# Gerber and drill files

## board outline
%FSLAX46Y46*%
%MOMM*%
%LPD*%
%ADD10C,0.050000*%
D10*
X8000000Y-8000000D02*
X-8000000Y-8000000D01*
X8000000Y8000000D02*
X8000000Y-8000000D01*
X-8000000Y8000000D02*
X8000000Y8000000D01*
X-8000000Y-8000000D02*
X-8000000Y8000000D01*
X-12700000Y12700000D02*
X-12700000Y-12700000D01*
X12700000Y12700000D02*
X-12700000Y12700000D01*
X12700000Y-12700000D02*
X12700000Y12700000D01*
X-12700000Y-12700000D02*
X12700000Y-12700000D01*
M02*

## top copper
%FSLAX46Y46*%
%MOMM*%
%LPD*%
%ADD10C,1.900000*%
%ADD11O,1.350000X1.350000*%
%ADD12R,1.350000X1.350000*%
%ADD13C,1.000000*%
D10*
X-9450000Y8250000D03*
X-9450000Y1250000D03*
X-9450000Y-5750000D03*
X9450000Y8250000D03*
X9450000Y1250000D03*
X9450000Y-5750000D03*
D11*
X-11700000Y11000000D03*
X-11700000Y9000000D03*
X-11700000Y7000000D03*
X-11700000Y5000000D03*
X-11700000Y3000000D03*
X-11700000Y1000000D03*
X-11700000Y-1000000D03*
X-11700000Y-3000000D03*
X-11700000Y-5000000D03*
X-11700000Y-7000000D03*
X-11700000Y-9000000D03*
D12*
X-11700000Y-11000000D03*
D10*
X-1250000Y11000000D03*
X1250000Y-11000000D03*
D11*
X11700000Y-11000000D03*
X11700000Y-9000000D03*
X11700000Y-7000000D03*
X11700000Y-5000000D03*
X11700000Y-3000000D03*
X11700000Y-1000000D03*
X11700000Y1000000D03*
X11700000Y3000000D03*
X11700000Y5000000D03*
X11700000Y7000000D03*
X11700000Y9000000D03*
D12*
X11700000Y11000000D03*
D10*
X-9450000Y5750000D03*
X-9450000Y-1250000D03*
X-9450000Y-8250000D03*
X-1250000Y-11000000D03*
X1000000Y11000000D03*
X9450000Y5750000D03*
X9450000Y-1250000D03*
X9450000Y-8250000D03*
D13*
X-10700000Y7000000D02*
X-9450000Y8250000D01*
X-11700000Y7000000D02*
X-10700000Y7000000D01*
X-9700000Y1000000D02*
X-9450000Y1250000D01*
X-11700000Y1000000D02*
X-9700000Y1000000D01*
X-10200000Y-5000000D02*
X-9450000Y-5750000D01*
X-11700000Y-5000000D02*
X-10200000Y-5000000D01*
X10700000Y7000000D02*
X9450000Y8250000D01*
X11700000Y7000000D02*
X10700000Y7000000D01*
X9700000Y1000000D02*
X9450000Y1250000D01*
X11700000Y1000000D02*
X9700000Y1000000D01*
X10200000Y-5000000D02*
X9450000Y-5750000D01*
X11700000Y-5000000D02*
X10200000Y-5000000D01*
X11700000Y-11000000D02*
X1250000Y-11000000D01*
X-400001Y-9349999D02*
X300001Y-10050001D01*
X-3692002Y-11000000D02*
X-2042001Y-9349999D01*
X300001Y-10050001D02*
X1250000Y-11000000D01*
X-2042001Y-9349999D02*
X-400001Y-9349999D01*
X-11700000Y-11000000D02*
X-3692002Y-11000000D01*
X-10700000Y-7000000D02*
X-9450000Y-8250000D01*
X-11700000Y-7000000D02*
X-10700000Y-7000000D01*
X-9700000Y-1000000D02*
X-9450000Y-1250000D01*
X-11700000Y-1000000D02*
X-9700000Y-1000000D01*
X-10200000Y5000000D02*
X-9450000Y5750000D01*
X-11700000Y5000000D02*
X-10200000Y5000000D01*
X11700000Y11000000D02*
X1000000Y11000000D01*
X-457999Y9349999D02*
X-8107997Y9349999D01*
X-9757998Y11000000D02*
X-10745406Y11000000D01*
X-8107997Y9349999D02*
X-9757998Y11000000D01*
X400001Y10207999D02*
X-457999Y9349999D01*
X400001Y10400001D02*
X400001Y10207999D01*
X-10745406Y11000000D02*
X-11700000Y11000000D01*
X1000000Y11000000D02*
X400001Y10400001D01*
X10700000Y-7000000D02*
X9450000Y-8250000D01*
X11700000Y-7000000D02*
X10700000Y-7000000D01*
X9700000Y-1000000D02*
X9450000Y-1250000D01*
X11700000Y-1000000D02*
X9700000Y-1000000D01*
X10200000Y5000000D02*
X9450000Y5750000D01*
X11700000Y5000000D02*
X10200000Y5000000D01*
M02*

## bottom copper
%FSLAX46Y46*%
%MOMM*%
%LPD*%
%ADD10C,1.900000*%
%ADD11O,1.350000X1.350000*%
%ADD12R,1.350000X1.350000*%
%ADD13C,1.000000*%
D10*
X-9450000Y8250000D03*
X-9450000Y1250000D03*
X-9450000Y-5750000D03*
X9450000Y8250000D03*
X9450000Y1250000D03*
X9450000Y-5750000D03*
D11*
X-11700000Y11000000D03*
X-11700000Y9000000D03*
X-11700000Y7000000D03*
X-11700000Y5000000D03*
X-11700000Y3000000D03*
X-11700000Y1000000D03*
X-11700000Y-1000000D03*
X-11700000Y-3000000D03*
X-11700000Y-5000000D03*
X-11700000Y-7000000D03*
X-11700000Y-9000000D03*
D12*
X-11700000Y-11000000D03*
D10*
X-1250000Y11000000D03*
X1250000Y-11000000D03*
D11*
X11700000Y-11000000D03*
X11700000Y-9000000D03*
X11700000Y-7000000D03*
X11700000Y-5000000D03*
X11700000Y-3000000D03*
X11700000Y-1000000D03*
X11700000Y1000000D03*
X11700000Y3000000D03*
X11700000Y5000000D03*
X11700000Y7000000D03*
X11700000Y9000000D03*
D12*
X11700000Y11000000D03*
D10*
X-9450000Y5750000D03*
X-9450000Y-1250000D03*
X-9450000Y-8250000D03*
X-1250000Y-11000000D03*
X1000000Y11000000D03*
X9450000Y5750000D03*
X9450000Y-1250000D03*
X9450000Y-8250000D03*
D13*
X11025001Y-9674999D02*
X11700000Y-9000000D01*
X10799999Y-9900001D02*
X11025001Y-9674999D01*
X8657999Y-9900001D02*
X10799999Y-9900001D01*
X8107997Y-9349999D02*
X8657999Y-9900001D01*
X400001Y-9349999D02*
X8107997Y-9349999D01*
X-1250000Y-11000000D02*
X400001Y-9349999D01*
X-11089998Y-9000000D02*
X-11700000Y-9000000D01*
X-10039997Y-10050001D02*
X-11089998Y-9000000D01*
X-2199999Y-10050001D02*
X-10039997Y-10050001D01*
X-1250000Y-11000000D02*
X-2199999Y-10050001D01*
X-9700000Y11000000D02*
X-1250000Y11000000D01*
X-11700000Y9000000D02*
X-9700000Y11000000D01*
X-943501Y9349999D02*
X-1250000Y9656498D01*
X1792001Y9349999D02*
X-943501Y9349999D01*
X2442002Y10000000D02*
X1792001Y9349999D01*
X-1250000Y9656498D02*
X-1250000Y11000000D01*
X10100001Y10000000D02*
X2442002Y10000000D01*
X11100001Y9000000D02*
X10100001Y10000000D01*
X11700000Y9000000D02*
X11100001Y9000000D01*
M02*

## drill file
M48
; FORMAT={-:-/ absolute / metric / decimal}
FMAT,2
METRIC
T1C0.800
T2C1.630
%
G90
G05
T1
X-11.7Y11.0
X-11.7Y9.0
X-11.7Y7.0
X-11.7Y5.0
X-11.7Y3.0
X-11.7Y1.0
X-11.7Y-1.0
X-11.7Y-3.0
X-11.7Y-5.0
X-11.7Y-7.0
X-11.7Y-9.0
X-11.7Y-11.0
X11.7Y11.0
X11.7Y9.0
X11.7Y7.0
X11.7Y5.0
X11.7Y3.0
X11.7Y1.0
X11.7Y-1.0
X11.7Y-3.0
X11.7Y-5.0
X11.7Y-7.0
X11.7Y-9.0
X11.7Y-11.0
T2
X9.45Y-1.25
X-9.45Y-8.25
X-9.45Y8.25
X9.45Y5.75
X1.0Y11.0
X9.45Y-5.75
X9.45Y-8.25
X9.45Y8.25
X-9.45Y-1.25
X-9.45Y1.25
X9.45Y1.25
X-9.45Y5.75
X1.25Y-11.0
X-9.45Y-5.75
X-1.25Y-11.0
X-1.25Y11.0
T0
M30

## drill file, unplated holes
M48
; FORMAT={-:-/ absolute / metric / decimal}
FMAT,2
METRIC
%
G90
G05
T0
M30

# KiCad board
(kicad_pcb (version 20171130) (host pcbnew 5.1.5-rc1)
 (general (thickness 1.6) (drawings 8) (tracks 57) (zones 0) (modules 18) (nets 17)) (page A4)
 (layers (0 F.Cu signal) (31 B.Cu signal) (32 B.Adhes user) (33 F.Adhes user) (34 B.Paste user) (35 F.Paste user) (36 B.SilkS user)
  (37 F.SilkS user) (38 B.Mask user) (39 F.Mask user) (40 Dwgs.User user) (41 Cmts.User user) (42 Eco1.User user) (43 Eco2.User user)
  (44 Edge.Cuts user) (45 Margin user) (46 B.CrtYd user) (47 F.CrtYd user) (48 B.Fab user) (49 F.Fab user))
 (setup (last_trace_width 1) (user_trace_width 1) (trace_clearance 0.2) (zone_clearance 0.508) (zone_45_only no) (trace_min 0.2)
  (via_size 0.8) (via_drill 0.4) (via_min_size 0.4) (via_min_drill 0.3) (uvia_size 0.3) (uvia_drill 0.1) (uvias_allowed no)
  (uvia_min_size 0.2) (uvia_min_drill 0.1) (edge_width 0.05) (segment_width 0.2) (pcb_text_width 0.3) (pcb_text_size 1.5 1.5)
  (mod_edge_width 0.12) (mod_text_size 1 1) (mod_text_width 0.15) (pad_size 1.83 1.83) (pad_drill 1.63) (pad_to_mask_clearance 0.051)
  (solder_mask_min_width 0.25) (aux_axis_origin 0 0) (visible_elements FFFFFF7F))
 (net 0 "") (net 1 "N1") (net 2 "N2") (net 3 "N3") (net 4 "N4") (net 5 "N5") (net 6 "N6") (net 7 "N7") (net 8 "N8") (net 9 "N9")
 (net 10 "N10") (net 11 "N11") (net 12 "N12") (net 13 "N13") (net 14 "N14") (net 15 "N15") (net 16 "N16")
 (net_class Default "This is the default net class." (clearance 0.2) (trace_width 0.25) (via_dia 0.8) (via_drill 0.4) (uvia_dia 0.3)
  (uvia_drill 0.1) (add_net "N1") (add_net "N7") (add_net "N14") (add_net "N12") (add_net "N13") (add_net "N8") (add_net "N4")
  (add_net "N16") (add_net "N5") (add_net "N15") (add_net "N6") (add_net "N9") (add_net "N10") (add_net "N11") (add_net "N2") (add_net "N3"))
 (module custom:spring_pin (layer F.Cu) (at -9.45 -8.25 90)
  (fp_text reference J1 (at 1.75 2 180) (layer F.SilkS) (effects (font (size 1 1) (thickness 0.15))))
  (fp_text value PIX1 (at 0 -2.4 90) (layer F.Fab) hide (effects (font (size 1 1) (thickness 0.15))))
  (pad 1 thru_hole circle (at 0 0 90) (size 1.9 1.9) (drill 1.63) (layers *.Cu *.Mask) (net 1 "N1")))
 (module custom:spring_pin (layer F.Cu) (at -9.45 -1.25 90)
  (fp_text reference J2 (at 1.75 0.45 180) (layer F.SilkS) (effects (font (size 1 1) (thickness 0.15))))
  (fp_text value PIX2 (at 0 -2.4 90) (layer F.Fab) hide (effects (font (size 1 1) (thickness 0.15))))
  (pad 1 thru_hole circle (at 0 0 90) (size 1.9 1.9) (drill 1.63) (layers *.Cu *.Mask) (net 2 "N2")))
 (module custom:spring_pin (layer F.Cu) (at -9.45 5.75 90)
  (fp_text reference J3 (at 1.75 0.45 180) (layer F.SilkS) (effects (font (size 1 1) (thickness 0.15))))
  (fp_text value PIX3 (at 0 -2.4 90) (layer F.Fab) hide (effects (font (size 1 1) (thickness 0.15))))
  (pad 1 thru_hole circle (at 0 0 90) (size 1.9 1.9) (drill 1.63) (layers *.Cu *.Mask) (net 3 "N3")))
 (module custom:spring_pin (layer F.Cu) (at 9.45 -8.25 90)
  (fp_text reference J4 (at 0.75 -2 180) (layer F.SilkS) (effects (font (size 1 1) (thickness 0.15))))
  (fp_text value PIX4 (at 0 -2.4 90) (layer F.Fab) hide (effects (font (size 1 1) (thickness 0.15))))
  (pad 1 thru_hole circle (at 0 0 90) (size 1.9 1.9) (drill 1.63) (layers *.Cu *.Mask) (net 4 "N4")))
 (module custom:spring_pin (layer F.Cu) (at 9.45 -1.25 90)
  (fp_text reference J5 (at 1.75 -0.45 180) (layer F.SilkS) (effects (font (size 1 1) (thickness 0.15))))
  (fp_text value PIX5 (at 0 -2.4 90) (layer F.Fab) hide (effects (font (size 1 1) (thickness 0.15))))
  (pad 1 thru_hole circle (at 0 0 90) (size 1.9 1.9) (drill 1.63) (layers *.Cu *.Mask) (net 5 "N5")))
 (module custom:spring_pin (layer F.Cu) (at 9.45 5.75 90)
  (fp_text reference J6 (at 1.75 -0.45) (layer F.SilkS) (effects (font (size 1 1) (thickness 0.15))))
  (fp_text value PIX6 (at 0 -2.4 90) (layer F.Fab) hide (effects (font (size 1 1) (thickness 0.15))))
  (pad 1 thru_hole circle (at 0 0 90) (size 1.9 1.9) (drill 1.63) (layers *.Cu *.Mask) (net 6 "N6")))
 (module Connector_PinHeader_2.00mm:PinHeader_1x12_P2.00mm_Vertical (layer B.Cu) (at -11.7 11)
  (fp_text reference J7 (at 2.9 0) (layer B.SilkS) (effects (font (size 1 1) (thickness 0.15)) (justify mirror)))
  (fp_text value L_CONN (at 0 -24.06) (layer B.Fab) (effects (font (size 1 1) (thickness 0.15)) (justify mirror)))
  (pad 12 thru_hole oval (at 0 -22) (size 1.35 1.35) (drill 0.8) (layers *.Cu *.Mask) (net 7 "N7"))
  (pad 11 thru_hole oval (at 0 -20) (size 1.35 1.35) (drill 0.8) (layers *.Cu *.Mask) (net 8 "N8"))
  (pad 10 thru_hole oval (at 0 -18) (size 1.35 1.35) (drill 0.8) (layers *.Cu *.Mask) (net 1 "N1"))
  (pad 9 thru_hole oval (at 0 -16) (size 1.35 1.35) (drill 0.8) (layers *.Cu *.Mask) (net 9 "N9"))
  (pad 8 thru_hole oval (at 0 -14) (size 1.35 1.35) (drill 0.8) (layers *.Cu *.Mask))
  (pad 7 thru_hole oval (at 0 -12) (size 1.35 1.35) (drill 0.8) (layers *.Cu *.Mask) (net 2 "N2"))
  (pad 6 thru_hole oval (at 0 -10) (size 1.35 1.35) (drill 0.8) (layers *.Cu *.Mask) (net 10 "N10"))
  (pad 5 thru_hole oval (at 0 -8) (size 1.35 1.35) (drill 0.8) (layers *.Cu *.Mask))
  (pad 4 thru_hole oval (at 0 -6) (size 1.35 1.35) (drill 0.8) (layers *.Cu *.Mask) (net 3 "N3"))
  (pad 3 thru_hole oval (at 0 -4) (size 1.35 1.35) (drill 0.8) (layers *.Cu *.Mask) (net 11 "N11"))
  (pad 2 thru_hole oval (at 0 -2) (size 1.35 1.35) (drill 0.8) (layers *.Cu *.Mask) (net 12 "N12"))
  (pad 1 thru_hole rect (at 0 0) (size 1.35 1.35) (drill 0.8) (layers *.Cu *.Mask) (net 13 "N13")))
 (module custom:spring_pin (layer F.Cu) (at -1.25 -11 90)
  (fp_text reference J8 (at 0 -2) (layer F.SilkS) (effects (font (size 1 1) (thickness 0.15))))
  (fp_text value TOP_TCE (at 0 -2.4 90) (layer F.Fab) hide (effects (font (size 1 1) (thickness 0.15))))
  (pad 1 thru_hole circle (at 0 0 90) (size 1.9 1.9) (drill 1.63) (layers *.Cu *.Mask) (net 8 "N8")))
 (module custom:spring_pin (layer F.Cu) (at 1.25 11 90)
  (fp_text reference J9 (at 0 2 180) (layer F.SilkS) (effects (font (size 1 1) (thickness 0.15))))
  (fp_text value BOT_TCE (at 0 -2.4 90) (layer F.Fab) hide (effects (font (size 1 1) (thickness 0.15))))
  (pad 1 thru_hole circle (at 0 0 90) (size 1.9 1.9) (drill 1.63) (layers *.Cu *.Mask) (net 13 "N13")))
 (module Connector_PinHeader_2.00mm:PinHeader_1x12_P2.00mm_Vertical (layer B.Cu) (at 11.7 -11 180)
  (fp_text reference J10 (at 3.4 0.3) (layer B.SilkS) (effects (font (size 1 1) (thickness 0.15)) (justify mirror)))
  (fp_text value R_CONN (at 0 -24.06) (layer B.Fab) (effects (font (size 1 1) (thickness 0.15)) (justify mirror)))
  (pad 12 thru_hole oval (at 0 -22 180) (size 1.35 1.35) (drill 0.8) (layers *.Cu *.Mask) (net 13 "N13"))
  (pad 11 thru_hole oval (at 0 -20 180) (size 1.35 1.35) (drill 0.8) (layers *.Cu *.Mask) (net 12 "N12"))
  (pad 10 thru_hole oval (at 0 -18 180) (size 1.35 1.35) (drill 0.8) (layers *.Cu *.Mask) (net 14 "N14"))
  (pad 9 thru_hole oval (at 0 -16 180) (size 1.35 1.35) (drill 0.8) (layers *.Cu *.Mask) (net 6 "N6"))
  (pad 8 thru_hole oval (at 0 -14 180) (size 1.35 1.35) (drill 0.8) (layers *.Cu *.Mask))
  (pad 7 thru_hole oval (at 0 -12 180) (size 1.35 1.35) (drill 0.8) (layers *.Cu *.Mask) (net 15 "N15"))
  (pad 6 thru_hole oval (at 0 -10 180) (size 1.35 1.35) (drill 0.8) (layers *.Cu *.Mask) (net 5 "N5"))
  (pad 5 thru_hole oval (at 0 -8 180) (size 1.35 1.35) (drill 0.8) (layers *.Cu *.Mask))
  (pad 4 thru_hole oval (at 0 -6 180) (size 1.35 1.35) (drill 0.8) (layers *.Cu *.Mask) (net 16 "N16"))
  (pad 3 thru_hole oval (at 0 -4 180) (size 1.35 1.35) (drill 0.8) (layers *.Cu *.Mask) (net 4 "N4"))
  (pad 2 thru_hole oval (at 0 -2 180) (size 1.35 1.35) (drill 0.8) (layers *.Cu *.Mask) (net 8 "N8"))
  (pad 1 thru_hole rect (at 0 0 180) (size 1.35 1.35) (drill 0.8) (layers *.Cu *.Mask) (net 7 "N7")))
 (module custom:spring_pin (layer F.Cu) (at -9.45 -5.75 90)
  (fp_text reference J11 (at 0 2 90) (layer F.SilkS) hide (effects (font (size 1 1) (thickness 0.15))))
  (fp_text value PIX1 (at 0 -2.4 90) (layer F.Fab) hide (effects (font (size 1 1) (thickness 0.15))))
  (pad 1 thru_hole circle (at 0 0 90) (size 1.9 1.9) (drill 1.63) (layers *.Cu *.Mask) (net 9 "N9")))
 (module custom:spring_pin (layer F.Cu) (at -9.45 1.25 90)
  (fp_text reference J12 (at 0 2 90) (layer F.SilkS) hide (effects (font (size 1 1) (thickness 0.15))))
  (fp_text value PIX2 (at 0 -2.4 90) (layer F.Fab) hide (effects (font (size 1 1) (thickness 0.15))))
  (pad 1 thru_hole circle (at 0 0 90) (size 1.9 1.9) (drill 1.63) (layers *.Cu *.Mask) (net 10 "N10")))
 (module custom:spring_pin (layer F.Cu) (at -9.45 8.25 90)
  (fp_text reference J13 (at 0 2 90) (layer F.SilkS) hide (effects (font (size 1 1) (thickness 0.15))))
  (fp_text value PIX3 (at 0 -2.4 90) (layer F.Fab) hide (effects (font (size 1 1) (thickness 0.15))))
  (pad 1 thru_hole circle (at 0 0 90) (size 1.9 1.9) (drill 1.63) (layers *.Cu *.Mask) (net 11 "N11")))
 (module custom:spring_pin (layer F.Cu) (at -1.25 11 90)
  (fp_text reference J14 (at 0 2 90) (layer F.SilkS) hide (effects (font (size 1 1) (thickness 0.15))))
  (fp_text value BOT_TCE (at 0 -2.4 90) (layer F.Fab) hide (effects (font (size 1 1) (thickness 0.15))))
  (pad 1 thru_hole circle (at 0 0 90) (size 1.9 1.9) (drill 1.63) (layers *.Cu *.Mask) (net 12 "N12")))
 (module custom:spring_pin (layer F.Cu) (at 1 -11 90)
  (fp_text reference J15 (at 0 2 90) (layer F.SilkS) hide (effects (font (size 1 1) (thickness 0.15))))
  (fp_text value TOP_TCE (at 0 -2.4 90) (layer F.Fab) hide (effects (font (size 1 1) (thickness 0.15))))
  (pad 1 thru_hole circle (at 0 0 90) (size 1.9 1.9) (drill 1.63) (layers *.Cu *.Mask) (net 7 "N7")))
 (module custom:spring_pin (layer F.Cu) (at 9.45 -5.75 90)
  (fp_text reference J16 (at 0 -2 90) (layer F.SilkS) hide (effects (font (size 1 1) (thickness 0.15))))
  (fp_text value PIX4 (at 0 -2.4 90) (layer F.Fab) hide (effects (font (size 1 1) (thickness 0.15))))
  (pad 1 thru_hole circle (at 0 0 90) (size 1.9 1.9) (drill 1.63) (layers *.Cu *.Mask) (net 16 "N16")))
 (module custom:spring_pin (layer F.Cu) (at 9.45 1.25 90)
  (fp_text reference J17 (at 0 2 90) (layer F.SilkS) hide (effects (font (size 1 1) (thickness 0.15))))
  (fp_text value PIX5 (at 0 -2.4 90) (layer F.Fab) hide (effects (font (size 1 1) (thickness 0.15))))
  (pad 1 thru_hole circle (at 0 0 90) (size 1.9 1.9) (drill 1.63) (layers *.Cu *.Mask) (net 15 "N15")))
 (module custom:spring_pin (layer F.Cu) (at 9.45 8.25 90)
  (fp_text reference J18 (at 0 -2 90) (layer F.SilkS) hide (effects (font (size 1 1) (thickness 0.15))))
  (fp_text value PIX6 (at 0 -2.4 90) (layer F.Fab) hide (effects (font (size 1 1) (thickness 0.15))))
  (pad 1 thru_hole circle (at 0 0 90) (size 1.9 1.9) (drill 1.63) (layers *.Cu *.Mask) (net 14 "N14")))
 (gr_line (start 8 8) (end -8 8) (layer Edge.Cuts) (width 0.05))
 (gr_line (start 8 -8) (end 8 8) (layer Edge.Cuts) (width 0.05))
 (gr_line (start -8 -8) (end 8 -8) (layer Edge.Cuts) (width 0.05))
 (gr_line (start -8 8) (end -8 -8) (layer Edge.Cuts) (width 0.05))
 (gr_line (start -12.7 -12.7) (end -12.7 12.7) (layer Edge.Cuts) (width 0.05))
 (gr_line (start 12.7 -12.7) (end -12.7 -12.7) (layer Edge.Cuts) (width 0.05))
 (gr_line (start 12.7 12.7) (end 12.7 -12.7) (layer Edge.Cuts) (width 0.05))
 (gr_line (start -12.7 12.7) (end 12.7 12.7) (layer Edge.Cuts) (width 0.05))
 (segment (start -10.7 -7) (end -9.45 -8.25) (width 1) (layer F.Cu) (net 1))
 (segment (start -11.7 -7) (end -10.7 -7) (width 1) (layer F.Cu) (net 1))
 (segment (start -9.7 -1) (end -9.45 -1.25) (width 1) (layer F.Cu) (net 2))
 (segment (start -11.7 -1) (end -9.7 -1) (width 1) (layer F.Cu) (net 2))
 (segment (start -10.2 5) (end -9.45 5.75) (width 1) (layer F.Cu) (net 3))
 (segment (start -11.7 5) (end -10.2 5) (width 1) (layer F.Cu) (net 3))
 (segment (start 10.7 -7) (end 9.45 -8.25) (width 1) (layer F.Cu) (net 4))
 (segment (start 11.7 -7) (end 10.7 -7) (width 1) (layer F.Cu) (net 4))
 (segment (start 9.7 -1) (end 9.45 -1.25) (width 1) (layer F.Cu) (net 5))
 (segment (start 11.7 -1) (end 9.7 -1) (width 1) (layer F.Cu) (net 5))
 (segment (start 10.2 5) (end 9.45 5.75) (width 1) (layer F.Cu) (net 6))
 (segment (start 11.7 5) (end 10.2 5) (width 1) (layer F.Cu) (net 6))
 (segment (start 11.7 11) (end 1.25 11) (width 1) (layer F.Cu) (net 13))
 (segment (start -0.400001 9.349999) (end 0.300001 10.050001) (width 1) (layer F.Cu) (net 13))
 (segment (start -3.692002 11) (end -2.042001 9.349999) (width 1) (layer F.Cu) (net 13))
 (segment (start 0.300001 10.050001) (end 1.25 11) (width 1) (layer F.Cu) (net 13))
 (segment (start -2.042001 9.349999) (end -0.400001 9.349999) (width 1) (layer F.Cu) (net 13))
 (segment (start -11.7 11) (end -3.692002 11) (width 1) (layer F.Cu) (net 13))
 (segment (start 11.025001 9.674999) (end 11.7 9) (width 1) (layer B.Cu) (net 12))
 (segment (start 10.799999 9.900001) (end 11.025001 9.674999) (width 1) (layer B.Cu) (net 12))
 (segment (start 8.657999 9.900001) (end 10.799999 9.900001) (width 1) (layer B.Cu) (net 12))
 (segment (start 8.107997 9.349999) (end 8.657999 9.900001) (width 1) (layer B.Cu) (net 12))
 (segment (start 0.400001 9.349999) (end 8.107997 9.349999) (width 1) (layer B.Cu) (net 12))
 (segment (start -1.25 11) (end 0.400001 9.349999) (width 1) (layer B.Cu) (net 12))
 (segment (start -11.089998 9) (end -11.7 9) (width 1) (layer B.Cu) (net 12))
 (segment (start -10.039997 10.050001) (end -11.089998 9) (width 1) (layer B.Cu) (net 12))
 (segment (start -2.199999 10.050001) (end -10.039997 10.050001) (width 1) (layer B.Cu) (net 12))
 (segment (start -1.25 11) (end -2.199999 10.050001) (width 1) (layer B.Cu) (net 12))
 (segment (start -10.7 7) (end -9.45 8.25) (width 1) (layer F.Cu) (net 11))
 (segment (start -11.7 7) (end -10.7 7) (width 1) (layer F.Cu) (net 11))
 (segment (start -9.7 1) (end -9.45 1.25) (width 1) (layer F.Cu) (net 10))
 (segment (start -11.7 1) (end -9.7 1) (width 1) (layer F.Cu) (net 10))
 (segment (start -10.2 -5) (end -9.45 -5.75) (width 1) (layer F.Cu) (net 9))
 (segment (start -11.7 -5) (end -10.2 -5) (width 1) (layer F.Cu) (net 9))
 (segment (start -9.7 -11) (end -1.25 -11) (width 1) (layer B.Cu) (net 8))
 (segment (start -11.7 -9) (end -9.7 -11) (width 1) (layer B.Cu) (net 8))
 (segment (start -0.943501 -9.349999) (end -1.25 -9.656498) (width 1) (layer B.Cu) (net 8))
 (segment (start 1.792001 -9.349999) (end -0.943501 -9.349999) (width 1) (layer B.Cu) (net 8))
 (segment (start 2.442002 -10) (end 1.792001 -9.349999) (width 1) (layer B.Cu) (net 8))
 (segment (start -1.25 -9.656498) (end -1.25 -11) (width 1) (layer B.Cu) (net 8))
 (segment (start 10.100001 -10) (end 2.442002 -10) (width 1) (layer B.Cu) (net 8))
 (segment (start 11.100001 -9) (end 10.100001 -10) (width 1) (layer B.Cu) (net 8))
 (segment (start 11.7 -9) (end 11.100001 -9) (width 1) (layer B.Cu) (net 8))
 (segment (start 11.7 -11) (end 1 -11) (width 1) (layer F.Cu) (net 7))
 (segment (start -0.457999 -9.349999) (end -8.107997 -9.349999) (width 1) (layer F.Cu) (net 7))
 (segment (start -9.757998 -11) (end -10.745406 -11) (width 1) (layer F.Cu) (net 7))
 (segment (start -8.107997 -9.349999) (end -9.757998 -11) (width 1) (layer F.Cu) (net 7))
 (segment (start 0.400001 -10.207999) (end -0.457999 -9.349999) (width 1) (layer F.Cu) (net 7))
 (segment (start 0.400001 -10.400001) (end 0.400001 -10.207999) (width 1) (layer F.Cu) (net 7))
 (segment (start -10.745406 -11) (end -11.7 -11) (width 1) (layer F.Cu) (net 7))
 (segment (start 1 -11) (end 0.400001 -10.400001) (width 1) (layer F.Cu) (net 7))
 (segment (start 10.7 7) (end 9.45 8.25) (width 1) (layer F.Cu) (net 14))
 (segment (start 11.7 7) (end 10.7 7) (width 1) (layer F.Cu) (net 14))
 (segment (start 9.7 1) (end 9.45 1.25) (width 1) (layer F.Cu) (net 15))
 (segment (start 11.7 1) (end 9.7 1) (width 1) (layer F.Cu) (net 15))
 (segment (start 10.2 -5) (end 9.45 -5.75) (width 1) (layer F.Cu) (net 16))
 (segment (start 11.7 -5) (end 10.2 -5) (width 1) (layer F.Cu) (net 16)))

